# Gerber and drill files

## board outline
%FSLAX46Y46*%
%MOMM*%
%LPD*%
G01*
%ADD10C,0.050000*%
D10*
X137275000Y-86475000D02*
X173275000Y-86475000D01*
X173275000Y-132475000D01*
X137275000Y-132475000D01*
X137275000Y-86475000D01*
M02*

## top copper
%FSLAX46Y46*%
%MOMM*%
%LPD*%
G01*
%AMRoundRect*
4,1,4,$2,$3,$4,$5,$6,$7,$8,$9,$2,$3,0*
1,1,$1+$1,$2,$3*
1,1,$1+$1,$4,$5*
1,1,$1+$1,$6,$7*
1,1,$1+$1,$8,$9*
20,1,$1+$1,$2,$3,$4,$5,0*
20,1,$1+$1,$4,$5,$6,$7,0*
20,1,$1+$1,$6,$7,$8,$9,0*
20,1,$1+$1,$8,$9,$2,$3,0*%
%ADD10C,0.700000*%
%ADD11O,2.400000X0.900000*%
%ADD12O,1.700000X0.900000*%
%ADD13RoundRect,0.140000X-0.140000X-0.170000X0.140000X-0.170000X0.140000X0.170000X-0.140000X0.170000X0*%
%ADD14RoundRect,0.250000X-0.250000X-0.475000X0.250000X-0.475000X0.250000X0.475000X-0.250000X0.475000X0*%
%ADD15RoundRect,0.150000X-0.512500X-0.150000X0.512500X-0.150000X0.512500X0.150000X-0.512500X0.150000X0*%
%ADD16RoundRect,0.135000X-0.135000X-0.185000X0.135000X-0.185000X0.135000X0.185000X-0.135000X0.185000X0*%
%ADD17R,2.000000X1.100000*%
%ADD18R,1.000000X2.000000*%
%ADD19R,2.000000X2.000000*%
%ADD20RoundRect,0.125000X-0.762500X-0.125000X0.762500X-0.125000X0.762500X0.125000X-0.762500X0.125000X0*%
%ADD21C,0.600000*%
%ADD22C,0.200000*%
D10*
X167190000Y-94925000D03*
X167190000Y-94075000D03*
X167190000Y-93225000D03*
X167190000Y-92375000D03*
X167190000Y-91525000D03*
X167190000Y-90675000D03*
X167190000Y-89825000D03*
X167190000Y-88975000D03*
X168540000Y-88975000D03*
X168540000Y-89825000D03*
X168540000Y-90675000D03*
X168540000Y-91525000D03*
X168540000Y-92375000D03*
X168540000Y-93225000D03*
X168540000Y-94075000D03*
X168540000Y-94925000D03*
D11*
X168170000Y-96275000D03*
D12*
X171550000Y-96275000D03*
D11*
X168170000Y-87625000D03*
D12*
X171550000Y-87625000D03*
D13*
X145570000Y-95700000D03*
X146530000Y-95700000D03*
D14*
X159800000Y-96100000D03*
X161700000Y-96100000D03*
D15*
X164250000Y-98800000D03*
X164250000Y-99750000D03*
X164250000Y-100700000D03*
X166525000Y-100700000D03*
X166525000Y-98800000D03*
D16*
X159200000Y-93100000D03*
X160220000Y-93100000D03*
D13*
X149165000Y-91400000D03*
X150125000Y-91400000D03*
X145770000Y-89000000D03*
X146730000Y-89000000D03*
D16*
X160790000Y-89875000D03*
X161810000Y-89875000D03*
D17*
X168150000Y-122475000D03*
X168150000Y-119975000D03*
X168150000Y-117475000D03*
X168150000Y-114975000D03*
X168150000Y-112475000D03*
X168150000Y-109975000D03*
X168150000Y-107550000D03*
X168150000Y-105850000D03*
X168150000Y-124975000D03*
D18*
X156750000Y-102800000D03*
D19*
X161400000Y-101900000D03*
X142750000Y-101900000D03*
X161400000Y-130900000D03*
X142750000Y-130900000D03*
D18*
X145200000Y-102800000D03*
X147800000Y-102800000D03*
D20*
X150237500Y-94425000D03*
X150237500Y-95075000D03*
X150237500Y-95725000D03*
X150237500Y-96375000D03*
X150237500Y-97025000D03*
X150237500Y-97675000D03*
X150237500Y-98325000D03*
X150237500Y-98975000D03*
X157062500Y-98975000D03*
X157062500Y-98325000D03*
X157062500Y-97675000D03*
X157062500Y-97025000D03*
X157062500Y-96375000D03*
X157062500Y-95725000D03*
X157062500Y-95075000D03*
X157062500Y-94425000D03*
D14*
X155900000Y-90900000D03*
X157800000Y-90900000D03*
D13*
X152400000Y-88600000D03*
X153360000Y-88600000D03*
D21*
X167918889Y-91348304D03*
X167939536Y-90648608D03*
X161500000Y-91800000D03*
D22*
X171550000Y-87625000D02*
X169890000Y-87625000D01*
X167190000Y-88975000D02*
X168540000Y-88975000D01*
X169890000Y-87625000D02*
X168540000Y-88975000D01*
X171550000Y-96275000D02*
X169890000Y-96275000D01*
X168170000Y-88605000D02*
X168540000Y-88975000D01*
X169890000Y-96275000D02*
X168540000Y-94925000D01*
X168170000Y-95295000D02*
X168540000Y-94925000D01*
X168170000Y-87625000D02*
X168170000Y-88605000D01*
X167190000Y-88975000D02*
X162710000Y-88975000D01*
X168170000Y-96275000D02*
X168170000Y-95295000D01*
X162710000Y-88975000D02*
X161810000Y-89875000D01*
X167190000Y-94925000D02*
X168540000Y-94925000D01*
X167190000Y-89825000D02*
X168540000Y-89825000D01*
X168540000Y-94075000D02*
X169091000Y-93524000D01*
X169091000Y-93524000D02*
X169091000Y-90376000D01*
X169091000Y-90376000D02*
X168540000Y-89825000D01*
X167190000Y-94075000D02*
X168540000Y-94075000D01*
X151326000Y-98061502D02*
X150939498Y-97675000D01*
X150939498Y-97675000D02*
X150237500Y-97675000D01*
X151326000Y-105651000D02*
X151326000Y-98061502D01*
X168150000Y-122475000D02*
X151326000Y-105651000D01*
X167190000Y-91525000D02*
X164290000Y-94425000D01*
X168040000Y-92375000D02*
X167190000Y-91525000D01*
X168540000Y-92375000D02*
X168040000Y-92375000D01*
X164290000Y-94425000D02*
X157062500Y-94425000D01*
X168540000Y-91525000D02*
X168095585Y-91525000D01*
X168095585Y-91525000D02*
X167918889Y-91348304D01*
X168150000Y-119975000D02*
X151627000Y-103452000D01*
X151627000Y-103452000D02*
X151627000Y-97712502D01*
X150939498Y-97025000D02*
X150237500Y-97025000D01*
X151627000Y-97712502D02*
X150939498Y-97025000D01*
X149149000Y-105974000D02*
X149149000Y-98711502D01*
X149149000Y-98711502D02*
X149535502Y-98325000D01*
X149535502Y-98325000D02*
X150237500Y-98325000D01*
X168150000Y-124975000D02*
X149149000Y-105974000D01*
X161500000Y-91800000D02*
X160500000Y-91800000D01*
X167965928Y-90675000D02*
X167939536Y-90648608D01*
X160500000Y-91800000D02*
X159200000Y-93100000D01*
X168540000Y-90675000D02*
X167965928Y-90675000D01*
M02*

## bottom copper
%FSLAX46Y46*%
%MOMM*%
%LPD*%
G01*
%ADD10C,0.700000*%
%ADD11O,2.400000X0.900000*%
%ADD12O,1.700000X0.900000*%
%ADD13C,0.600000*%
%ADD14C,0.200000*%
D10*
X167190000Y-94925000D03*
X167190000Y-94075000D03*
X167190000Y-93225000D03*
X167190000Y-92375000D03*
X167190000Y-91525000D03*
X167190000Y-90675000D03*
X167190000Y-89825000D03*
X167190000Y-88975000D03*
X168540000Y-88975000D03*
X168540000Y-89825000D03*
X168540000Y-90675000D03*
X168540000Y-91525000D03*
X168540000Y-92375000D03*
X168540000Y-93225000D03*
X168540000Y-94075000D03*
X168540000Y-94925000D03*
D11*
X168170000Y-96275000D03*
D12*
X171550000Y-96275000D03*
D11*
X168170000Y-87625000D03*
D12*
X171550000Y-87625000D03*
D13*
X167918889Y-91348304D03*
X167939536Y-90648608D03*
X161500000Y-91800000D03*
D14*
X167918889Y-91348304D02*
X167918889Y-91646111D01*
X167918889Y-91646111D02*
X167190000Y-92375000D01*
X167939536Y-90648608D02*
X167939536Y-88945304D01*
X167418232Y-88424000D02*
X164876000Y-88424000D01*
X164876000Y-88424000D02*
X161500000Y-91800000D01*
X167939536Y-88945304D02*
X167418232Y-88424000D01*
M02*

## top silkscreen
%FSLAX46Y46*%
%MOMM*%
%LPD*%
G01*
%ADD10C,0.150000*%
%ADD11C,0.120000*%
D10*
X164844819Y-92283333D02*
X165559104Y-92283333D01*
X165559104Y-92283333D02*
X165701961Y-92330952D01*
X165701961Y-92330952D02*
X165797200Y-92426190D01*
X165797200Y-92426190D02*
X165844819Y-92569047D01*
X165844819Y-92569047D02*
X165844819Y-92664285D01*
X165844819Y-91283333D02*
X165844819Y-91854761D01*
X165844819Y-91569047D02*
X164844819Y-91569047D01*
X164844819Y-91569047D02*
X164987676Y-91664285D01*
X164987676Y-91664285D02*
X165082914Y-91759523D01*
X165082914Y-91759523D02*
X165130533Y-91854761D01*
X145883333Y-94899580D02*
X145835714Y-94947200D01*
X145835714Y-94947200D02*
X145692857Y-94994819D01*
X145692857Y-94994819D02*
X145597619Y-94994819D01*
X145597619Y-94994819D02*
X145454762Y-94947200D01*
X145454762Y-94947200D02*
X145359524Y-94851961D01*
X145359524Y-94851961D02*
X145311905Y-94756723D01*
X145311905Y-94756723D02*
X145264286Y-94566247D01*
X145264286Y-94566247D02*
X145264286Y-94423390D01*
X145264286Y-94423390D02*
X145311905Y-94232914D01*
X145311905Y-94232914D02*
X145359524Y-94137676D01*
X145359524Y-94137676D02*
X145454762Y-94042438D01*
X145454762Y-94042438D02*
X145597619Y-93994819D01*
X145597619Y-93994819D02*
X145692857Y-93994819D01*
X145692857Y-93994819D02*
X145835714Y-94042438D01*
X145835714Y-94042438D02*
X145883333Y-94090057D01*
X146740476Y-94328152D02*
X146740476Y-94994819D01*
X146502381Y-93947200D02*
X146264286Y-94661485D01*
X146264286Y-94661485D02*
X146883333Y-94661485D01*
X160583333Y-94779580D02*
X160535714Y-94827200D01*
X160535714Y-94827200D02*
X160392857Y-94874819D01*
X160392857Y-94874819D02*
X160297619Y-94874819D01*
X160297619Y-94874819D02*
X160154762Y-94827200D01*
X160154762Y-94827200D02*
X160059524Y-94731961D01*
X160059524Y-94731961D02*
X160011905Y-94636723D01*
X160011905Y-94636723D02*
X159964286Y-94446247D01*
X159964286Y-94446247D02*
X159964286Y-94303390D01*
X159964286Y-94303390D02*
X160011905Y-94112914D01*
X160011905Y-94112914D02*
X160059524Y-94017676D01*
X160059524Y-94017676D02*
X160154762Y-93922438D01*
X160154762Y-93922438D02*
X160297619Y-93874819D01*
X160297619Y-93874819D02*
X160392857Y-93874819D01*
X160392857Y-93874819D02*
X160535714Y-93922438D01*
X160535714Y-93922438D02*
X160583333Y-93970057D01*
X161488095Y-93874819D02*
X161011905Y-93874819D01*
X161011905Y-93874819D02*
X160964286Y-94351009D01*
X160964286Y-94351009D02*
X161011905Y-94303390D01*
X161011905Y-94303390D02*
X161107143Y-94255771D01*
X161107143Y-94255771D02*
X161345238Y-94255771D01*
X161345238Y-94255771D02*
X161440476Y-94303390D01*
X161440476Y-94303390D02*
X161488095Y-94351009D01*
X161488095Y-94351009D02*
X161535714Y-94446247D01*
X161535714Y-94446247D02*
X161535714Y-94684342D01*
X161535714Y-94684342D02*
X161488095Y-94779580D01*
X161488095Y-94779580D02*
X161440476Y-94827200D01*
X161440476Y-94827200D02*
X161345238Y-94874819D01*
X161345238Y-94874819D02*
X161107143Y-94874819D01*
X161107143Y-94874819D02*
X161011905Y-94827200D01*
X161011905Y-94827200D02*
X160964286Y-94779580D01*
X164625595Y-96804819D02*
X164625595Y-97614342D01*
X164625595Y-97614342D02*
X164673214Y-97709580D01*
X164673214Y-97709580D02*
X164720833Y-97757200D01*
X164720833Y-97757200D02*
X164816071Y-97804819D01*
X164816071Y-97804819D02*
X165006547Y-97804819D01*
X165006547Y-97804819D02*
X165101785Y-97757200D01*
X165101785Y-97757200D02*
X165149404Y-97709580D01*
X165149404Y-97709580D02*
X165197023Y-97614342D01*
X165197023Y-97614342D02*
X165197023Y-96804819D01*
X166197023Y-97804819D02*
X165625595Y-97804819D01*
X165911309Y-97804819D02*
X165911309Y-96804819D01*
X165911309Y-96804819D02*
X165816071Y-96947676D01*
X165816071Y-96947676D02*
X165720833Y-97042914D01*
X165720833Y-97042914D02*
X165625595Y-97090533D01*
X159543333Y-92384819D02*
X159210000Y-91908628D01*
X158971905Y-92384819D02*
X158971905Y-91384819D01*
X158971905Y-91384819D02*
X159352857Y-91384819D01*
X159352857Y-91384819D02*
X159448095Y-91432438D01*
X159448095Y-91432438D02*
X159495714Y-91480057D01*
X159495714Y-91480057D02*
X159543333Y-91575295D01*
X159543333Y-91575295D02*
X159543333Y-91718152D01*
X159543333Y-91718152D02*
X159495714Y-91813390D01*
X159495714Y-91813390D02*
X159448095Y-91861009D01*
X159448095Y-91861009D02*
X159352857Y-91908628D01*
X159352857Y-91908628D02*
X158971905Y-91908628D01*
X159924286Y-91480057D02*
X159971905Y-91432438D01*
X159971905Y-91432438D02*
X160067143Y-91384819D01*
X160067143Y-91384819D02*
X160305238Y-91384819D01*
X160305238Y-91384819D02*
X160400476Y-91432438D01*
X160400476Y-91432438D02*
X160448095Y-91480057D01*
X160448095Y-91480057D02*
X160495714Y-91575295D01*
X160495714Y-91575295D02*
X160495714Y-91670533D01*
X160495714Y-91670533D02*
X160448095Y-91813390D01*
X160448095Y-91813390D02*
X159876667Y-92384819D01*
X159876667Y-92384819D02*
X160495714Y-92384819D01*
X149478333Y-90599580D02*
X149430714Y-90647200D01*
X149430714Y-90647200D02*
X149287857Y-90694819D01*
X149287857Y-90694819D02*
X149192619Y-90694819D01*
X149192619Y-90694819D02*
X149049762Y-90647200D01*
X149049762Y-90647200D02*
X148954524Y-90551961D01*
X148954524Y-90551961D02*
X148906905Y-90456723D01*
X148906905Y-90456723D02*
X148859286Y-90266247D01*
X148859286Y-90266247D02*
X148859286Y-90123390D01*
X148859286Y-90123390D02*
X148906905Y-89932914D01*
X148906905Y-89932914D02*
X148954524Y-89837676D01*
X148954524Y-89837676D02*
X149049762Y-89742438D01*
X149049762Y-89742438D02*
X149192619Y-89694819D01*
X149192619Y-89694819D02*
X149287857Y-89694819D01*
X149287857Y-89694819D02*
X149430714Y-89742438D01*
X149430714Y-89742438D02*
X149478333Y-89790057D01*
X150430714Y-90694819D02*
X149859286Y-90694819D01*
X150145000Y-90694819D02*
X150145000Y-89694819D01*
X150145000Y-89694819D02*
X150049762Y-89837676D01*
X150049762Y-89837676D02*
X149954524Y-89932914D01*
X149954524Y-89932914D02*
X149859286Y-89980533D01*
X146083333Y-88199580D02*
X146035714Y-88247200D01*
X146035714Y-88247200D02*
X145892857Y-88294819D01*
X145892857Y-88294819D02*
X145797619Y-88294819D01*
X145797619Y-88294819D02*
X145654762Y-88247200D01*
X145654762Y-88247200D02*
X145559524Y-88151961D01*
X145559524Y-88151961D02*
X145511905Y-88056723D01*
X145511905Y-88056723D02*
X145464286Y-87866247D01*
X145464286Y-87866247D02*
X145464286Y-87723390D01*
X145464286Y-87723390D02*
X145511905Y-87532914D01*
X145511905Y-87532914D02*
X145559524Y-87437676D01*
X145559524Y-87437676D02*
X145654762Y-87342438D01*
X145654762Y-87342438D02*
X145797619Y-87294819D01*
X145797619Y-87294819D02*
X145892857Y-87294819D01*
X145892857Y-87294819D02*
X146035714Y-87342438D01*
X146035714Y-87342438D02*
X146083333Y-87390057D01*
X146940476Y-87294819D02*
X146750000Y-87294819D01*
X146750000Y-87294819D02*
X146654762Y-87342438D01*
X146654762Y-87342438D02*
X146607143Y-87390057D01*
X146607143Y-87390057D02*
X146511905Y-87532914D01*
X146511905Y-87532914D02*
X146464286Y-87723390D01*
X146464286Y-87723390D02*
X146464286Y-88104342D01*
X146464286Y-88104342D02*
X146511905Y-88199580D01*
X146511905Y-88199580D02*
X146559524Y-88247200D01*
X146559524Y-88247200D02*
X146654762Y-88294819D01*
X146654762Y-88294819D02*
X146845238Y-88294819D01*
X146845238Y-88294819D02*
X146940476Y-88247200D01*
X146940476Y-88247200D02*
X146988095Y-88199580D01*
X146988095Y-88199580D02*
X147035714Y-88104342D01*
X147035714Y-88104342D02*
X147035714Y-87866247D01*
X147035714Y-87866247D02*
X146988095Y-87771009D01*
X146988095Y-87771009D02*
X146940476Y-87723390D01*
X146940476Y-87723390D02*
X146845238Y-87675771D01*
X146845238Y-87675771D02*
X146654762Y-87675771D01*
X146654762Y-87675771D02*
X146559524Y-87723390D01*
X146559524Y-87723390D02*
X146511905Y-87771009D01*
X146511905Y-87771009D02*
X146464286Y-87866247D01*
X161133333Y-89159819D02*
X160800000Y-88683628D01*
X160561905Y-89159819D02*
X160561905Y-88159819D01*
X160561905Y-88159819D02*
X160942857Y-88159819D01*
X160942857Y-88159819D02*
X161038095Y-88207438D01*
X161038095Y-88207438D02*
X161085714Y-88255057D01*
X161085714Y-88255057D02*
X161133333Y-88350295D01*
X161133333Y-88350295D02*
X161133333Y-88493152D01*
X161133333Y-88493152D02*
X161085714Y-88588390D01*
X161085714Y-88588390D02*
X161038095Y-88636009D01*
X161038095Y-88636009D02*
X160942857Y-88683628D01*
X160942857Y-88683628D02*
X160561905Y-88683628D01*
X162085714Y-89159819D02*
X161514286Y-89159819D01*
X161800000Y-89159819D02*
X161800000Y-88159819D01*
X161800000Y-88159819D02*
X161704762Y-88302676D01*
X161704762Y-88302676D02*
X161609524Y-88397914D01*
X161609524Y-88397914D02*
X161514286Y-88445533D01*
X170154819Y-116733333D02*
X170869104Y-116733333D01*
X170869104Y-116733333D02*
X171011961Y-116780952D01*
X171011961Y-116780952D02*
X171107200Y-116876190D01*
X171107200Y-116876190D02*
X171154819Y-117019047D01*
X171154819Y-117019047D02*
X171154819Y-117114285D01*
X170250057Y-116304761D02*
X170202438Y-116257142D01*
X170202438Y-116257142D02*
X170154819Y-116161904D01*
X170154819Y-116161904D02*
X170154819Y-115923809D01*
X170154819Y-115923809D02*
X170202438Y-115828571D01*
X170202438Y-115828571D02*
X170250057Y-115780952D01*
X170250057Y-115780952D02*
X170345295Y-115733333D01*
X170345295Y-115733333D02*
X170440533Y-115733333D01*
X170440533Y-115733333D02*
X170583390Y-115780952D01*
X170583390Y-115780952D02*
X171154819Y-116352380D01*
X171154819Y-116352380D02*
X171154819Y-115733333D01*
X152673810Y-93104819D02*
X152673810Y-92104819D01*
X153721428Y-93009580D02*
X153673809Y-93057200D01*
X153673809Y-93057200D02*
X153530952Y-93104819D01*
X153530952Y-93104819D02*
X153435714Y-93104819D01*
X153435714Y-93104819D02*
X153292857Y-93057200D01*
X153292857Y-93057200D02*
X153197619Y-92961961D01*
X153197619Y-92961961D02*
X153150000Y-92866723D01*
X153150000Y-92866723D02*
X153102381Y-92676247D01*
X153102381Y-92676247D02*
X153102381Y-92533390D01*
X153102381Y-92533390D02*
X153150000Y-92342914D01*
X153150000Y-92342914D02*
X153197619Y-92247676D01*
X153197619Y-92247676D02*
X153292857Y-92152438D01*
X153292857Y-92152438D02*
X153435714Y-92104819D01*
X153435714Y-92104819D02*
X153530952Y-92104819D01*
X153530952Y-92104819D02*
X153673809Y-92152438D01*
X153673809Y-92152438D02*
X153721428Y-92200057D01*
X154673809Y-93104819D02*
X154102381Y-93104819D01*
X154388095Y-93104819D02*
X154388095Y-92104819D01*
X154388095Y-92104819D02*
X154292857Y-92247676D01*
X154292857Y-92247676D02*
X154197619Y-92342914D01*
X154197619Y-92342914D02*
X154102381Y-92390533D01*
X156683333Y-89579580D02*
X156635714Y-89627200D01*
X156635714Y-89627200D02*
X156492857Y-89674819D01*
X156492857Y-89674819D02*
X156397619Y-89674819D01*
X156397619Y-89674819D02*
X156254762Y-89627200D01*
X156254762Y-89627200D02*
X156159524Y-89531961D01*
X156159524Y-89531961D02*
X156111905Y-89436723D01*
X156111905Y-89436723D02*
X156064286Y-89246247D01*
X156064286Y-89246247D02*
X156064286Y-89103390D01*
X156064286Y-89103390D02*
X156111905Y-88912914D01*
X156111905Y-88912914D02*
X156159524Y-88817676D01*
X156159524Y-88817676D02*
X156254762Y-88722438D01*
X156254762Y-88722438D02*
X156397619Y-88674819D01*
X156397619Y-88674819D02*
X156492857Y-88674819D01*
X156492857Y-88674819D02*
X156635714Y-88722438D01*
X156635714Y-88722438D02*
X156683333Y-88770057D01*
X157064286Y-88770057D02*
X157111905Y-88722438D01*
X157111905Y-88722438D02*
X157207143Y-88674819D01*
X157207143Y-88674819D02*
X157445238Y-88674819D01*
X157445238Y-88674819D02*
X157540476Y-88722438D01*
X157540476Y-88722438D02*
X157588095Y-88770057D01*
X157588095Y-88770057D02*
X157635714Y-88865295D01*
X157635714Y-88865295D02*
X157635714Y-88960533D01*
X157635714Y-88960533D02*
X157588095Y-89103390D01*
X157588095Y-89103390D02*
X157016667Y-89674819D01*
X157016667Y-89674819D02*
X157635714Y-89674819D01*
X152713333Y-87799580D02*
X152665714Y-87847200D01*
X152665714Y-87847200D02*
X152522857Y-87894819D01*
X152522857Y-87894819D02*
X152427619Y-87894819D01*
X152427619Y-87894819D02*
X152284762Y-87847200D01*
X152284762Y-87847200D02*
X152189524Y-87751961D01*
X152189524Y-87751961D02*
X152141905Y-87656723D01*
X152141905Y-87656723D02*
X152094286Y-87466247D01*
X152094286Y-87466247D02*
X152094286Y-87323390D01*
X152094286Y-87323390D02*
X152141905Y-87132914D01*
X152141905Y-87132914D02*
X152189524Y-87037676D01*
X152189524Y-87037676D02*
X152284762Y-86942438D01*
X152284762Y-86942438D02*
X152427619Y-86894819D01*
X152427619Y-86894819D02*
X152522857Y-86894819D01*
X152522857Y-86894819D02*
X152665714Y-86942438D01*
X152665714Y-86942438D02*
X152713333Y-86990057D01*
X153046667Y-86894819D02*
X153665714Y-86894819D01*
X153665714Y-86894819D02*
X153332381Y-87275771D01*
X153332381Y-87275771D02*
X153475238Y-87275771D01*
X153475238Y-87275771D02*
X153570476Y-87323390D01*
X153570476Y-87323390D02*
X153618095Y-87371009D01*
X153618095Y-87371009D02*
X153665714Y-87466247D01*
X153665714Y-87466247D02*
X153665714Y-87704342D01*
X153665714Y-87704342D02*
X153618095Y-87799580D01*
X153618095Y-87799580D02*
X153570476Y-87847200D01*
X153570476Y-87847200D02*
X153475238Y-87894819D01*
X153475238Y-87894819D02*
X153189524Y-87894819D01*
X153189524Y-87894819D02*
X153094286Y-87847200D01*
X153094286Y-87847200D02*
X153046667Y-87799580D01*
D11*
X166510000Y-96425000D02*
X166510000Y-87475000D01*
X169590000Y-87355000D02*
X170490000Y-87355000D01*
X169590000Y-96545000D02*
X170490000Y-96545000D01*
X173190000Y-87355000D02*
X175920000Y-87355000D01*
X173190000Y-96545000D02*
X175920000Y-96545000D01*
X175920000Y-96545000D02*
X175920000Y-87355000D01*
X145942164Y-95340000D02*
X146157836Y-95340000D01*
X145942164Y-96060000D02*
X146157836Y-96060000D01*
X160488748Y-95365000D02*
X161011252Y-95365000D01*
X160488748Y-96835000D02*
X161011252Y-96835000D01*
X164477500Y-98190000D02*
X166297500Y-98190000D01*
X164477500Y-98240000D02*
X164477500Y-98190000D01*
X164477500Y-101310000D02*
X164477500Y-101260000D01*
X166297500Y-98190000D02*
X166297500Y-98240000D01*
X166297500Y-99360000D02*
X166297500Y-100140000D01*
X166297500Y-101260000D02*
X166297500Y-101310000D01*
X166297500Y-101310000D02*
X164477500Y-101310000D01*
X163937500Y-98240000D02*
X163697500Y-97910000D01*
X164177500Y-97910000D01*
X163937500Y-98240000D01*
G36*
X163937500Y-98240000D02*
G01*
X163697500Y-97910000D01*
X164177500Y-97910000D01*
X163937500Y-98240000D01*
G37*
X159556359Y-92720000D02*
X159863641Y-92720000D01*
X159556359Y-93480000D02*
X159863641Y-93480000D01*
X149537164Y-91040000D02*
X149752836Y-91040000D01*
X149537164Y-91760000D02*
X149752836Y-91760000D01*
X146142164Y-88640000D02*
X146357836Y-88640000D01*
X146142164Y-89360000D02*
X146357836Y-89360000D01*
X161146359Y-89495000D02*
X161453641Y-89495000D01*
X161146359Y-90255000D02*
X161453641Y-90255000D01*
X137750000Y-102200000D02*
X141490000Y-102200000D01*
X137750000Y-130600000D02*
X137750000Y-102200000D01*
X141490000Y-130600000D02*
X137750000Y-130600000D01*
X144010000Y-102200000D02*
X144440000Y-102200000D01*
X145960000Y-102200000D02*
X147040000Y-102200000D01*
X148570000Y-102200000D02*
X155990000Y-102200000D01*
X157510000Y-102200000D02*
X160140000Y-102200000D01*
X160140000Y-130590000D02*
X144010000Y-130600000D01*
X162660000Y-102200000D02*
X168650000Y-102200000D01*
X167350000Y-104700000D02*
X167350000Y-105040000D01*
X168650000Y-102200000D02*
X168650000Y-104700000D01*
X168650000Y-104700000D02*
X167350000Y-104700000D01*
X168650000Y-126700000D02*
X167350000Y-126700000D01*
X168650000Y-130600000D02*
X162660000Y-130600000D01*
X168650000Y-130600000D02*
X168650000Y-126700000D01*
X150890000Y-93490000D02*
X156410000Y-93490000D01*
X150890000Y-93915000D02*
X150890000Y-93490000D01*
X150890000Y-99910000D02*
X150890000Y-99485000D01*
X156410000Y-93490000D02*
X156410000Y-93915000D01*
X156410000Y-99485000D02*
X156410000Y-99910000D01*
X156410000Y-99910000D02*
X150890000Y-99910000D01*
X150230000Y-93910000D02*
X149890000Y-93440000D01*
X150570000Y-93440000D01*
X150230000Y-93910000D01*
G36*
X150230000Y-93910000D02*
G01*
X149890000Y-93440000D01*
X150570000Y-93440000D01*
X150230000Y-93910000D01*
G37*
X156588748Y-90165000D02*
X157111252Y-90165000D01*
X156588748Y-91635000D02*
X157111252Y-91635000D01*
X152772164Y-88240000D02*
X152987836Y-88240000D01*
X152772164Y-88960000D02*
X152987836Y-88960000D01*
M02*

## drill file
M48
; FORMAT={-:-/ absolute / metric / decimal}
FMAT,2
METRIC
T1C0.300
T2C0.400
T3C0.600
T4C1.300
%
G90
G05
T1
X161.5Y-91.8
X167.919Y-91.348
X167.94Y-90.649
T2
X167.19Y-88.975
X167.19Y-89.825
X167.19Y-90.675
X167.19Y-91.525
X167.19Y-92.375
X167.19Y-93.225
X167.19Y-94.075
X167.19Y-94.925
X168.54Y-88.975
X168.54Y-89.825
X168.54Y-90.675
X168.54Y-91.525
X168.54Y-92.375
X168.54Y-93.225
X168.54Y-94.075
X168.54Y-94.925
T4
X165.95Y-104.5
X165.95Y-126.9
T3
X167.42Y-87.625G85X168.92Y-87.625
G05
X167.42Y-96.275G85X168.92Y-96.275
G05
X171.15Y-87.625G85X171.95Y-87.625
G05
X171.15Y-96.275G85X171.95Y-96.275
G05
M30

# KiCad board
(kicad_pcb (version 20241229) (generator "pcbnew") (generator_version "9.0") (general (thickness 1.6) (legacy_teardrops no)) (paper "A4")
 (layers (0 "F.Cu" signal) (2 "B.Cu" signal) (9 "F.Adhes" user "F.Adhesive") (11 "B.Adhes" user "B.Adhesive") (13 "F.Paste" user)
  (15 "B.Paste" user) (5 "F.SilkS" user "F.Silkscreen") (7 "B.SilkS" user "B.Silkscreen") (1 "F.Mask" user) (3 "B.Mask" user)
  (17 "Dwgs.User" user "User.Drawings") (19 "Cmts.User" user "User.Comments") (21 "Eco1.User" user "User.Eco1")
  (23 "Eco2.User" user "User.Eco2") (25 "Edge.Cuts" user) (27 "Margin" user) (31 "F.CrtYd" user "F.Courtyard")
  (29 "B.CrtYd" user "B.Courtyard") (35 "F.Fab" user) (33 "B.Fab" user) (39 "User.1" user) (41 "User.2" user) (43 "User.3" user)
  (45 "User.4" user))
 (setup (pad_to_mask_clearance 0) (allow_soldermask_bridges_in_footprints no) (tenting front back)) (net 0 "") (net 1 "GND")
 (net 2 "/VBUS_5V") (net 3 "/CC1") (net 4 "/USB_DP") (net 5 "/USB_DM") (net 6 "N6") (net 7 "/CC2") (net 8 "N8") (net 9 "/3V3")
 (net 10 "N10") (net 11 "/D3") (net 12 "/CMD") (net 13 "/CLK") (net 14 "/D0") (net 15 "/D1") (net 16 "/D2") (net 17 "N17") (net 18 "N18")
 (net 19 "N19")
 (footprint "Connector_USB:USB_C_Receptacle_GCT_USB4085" (layer "F.Cu") (at 167.19 94.925 90)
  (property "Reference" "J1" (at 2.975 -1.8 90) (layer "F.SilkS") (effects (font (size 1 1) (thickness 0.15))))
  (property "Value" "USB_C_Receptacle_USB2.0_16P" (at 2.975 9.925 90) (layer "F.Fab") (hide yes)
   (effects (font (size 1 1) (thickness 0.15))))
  (fp_line (start -1.5 -0.68) (end 7.45 -0.68) (stroke (width 0.12) (type solid)) (layer "F.SilkS"))
  (fp_line (start 7.57 2.4) (end 7.57 3.3) (stroke (width 0.12) (type solid)) (layer "F.SilkS"))
  (fp_line (start -1.62 2.4) (end -1.62 3.3) (stroke (width 0.12) (type solid)) (layer "F.SilkS"))
  (fp_line (start 7.57 6) (end 7.57 8.73) (stroke (width 0.12) (type solid)) (layer "F.SilkS"))
  (fp_line (start -1.62 6) (end -1.62 8.73) (stroke (width 0.12) (type solid)) (layer "F.SilkS"))
  (fp_line (start -1.62 8.73) (end 7.57 8.73) (stroke (width 0.12) (type solid)) (layer "F.SilkS"))
  (pad "A1" thru_hole circle (at 0 0 90) (size 0.7 0.7) (drill 0.4) (layers "*.Cu" "*.Mask") (remove_unused_layers no) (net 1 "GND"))
  (pad "A4" thru_hole circle (at 0.85 0 90) (size 0.7 0.7) (drill 0.4) (layers "*.Cu" "*.Mask") (remove_unused_layers no) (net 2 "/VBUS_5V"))
  (pad "A5" thru_hole circle (at 1.7 0 90) (size 0.7 0.7) (drill 0.4) (layers "*.Cu" "*.Mask") (remove_unused_layers no) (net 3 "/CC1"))
  (pad "A6" thru_hole circle (at 2.55 0 90) (size 0.7 0.7) (drill 0.4) (layers "*.Cu" "*.Mask") (remove_unused_layers no) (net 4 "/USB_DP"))
  (pad "A7" thru_hole circle (at 3.4 0 90) (size 0.7 0.7) (drill 0.4) (layers "*.Cu" "*.Mask") (remove_unused_layers no) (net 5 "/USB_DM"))
  (pad "A8" thru_hole circle (at 4.25 0 90) (size 0.7 0.7) (drill 0.4) (layers "*.Cu" "*.Mask") (remove_unused_layers no) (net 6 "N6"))
  (pad "A9" thru_hole circle (at 5.1 0 90) (size 0.7 0.7) (drill 0.4) (layers "*.Cu" "*.Mask") (remove_unused_layers no) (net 2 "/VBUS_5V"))
  (pad "A12" thru_hole circle (at 5.95 0 90) (size 0.7 0.7) (drill 0.4) (layers "*.Cu" "*.Mask") (remove_unused_layers no) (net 1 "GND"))
  (pad "B1" thru_hole circle (at 5.95 1.35 90) (size 0.7 0.7) (drill 0.4) (layers "*.Cu" "*.Mask") (remove_unused_layers no) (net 1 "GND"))
  (pad "B4" thru_hole circle (at 5.1 1.35 90) (size 0.7 0.7) (drill 0.4) (layers "*.Cu" "*.Mask") (remove_unused_layers no)
   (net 2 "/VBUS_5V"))
  (pad "B5" thru_hole circle (at 4.25 1.35 90) (size 0.7 0.7) (drill 0.4) (layers "*.Cu" "*.Mask") (remove_unused_layers no) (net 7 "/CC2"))
  (pad "B6" thru_hole circle (at 3.4 1.35 90) (size 0.7 0.7) (drill 0.4) (layers "*.Cu" "*.Mask") (remove_unused_layers no)
   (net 4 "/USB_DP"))
  (pad "B7" thru_hole circle (at 2.55 1.35 90) (size 0.7 0.7) (drill 0.4) (layers "*.Cu" "*.Mask") (remove_unused_layers no)
   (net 5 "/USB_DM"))
  (pad "B8" thru_hole circle (at 1.7 1.35 90) (size 0.7 0.7) (drill 0.4) (layers "*.Cu" "*.Mask") (remove_unused_layers no) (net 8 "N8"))
  (pad "B9" thru_hole circle (at 0.85 1.35 90) (size 0.7 0.7) (drill 0.4) (layers "*.Cu" "*.Mask") (remove_unused_layers no)
   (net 2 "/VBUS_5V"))
  (pad "B12" thru_hole circle (at 0 1.35 90) (size 0.7 0.7) (drill 0.4) (layers "*.Cu" "*.Mask") (remove_unused_layers no) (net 1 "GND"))
  (pad "S1" thru_hole oval (at -1.35 0.98 90) (size 0.9 2.4) (drill oval 0.6 2.1) (layers "*.Cu" "*.Mask") (remove_unused_layers no)
   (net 1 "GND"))
  (pad "S1" thru_hole oval (at -1.35 4.36 90) (size 0.9 1.7) (drill oval 0.6 1.4) (layers "*.Cu" "*.Mask") (remove_unused_layers no)
   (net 1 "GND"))
  (pad "S1" thru_hole oval (at 7.3 0.98 90) (size 0.9 2.4) (drill oval 0.6 2.1) (layers "*.Cu" "*.Mask") (remove_unused_layers no)
   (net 1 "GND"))
  (pad "S1" thru_hole oval (at 7.3 4.36 90) (size 0.9 1.7) (drill oval 0.6 1.4) (layers "*.Cu" "*.Mask") (remove_unused_layers no)
   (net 1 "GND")))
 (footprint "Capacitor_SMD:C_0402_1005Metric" (layer "F.Cu") (at 146.05 95.7)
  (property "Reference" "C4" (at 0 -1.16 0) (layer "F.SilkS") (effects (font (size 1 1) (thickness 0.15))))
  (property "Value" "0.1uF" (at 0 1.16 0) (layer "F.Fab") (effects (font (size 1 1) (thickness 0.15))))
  (fp_line (start -0.107836 -0.36) (end 0.107836 -0.36) (stroke (width 0.12) (type solid)) (layer "F.SilkS"))
  (fp_line (start -0.107836 0.36) (end 0.107836 0.36) (stroke (width 0.12) (type solid)) (layer "F.SilkS"))
  (pad "1" smd roundrect (at -0.48 0) (size 0.56 0.62) (layers "F.Cu" "F.Mask" "F.Paste") (roundrect_rratio 0.25) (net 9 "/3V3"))
  (pad "2" smd roundrect (at 0.48 0) (size 0.56 0.62) (layers "F.Cu" "F.Mask" "F.Paste") (roundrect_rratio 0.25) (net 1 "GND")))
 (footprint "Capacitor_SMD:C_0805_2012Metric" (layer "F.Cu") (at 160.75 96.1)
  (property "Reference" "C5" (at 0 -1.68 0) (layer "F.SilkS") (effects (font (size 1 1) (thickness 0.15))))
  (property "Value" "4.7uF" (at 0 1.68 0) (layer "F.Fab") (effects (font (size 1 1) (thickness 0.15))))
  (fp_line (start -0.261252 -0.735) (end 0.261252 -0.735) (stroke (width 0.12) (type solid)) (layer "F.SilkS"))
  (fp_line (start -0.261252 0.735) (end 0.261252 0.735) (stroke (width 0.12) (type solid)) (layer "F.SilkS"))
  (pad "1" smd roundrect (at -0.95 0) (size 1 1.45) (layers "F.Cu" "F.Mask" "F.Paste") (roundrect_rratio 0.25) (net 9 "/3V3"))
  (pad "2" smd roundrect (at 0.95 0) (size 1 1.45) (layers "F.Cu" "F.Mask" "F.Paste") (roundrect_rratio 0.25) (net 1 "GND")))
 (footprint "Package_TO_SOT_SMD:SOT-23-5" (layer "F.Cu") (at 165.3875 99.75)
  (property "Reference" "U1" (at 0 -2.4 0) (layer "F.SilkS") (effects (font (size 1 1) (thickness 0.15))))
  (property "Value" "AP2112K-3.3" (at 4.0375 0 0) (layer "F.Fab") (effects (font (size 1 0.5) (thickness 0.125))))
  (fp_line (start -0.91 -1.56) (end 0.91 -1.56) (stroke (width 0.12) (type solid)) (layer "F.SilkS"))
  (fp_line (start -0.91 -1.51) (end -0.91 -1.56) (stroke (width 0.12) (type solid)) (layer "F.SilkS"))
  (fp_line (start -0.91 1.56) (end -0.91 1.51) (stroke (width 0.12) (type solid)) (layer "F.SilkS"))
  (fp_line (start 0.91 -1.56) (end 0.91 -1.51) (stroke (width 0.12) (type solid)) (layer "F.SilkS"))
  (fp_line (start 0.91 -0.39) (end 0.91 0.39) (stroke (width 0.12) (type solid)) (layer "F.SilkS"))
  (fp_line (start 0.91 1.51) (end 0.91 1.56) (stroke (width 0.12) (type solid)) (layer "F.SilkS"))
  (fp_line (start 0.91 1.56) (end -0.91 1.56) (stroke (width 0.12) (type solid)) (layer "F.SilkS"))
  (fp_poly (pts (xy -1.45 -1.51) (xy -1.69 -1.84) (xy -1.21 -1.84)) (stroke (width 0.12) (type solid)) (fill yes) (layer "F.SilkS"))
  (pad "1" smd roundrect (at -1.1375 -0.95) (size 1.325 0.6) (layers "F.Cu" "F.Mask" "F.Paste") (roundrect_rratio 0.25) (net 2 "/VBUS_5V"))
  (pad "2" smd roundrect (at -1.1375 0) (size 1.325 0.6) (layers "F.Cu" "F.Mask" "F.Paste") (roundrect_rratio 0.25) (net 1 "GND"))
  (pad "3" smd roundrect (at -1.1375 0.95) (size 1.325 0.6) (layers "F.Cu" "F.Mask" "F.Paste") (roundrect_rratio 0.25) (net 2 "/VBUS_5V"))
  (pad "4" smd roundrect (at 1.1375 0.95) (size 1.325 0.6) (layers "F.Cu" "F.Mask" "F.Paste") (roundrect_rratio 0.25) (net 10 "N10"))
  (pad "5" smd roundrect (at 1.1375 -0.95) (size 1.325 0.6) (layers "F.Cu" "F.Mask" "F.Paste") (roundrect_rratio 0.25) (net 9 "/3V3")))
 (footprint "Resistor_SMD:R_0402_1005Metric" (layer "F.Cu") (at 159.71 93.1)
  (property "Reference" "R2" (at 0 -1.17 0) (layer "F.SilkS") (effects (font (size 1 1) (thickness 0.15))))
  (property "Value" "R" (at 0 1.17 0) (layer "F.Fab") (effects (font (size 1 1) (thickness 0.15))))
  (fp_line (start -0.153641 -0.38) (end 0.153641 -0.38) (stroke (width 0.12) (type solid)) (layer "F.SilkS"))
  (fp_line (start -0.153641 0.38) (end 0.153641 0.38) (stroke (width 0.12) (type solid)) (layer "F.SilkS"))
  (pad "1" smd roundrect (at -0.51 0) (size 0.54 0.64) (layers "F.Cu" "F.Mask" "F.Paste") (roundrect_rratio 0.25) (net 7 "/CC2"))
  (pad "2" smd roundrect (at 0.51 0) (size 0.54 0.64) (layers "F.Cu" "F.Mask" "F.Paste") (roundrect_rratio 0.25) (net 1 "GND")))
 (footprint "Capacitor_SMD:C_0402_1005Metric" (layer "F.Cu") (at 149.645 91.4)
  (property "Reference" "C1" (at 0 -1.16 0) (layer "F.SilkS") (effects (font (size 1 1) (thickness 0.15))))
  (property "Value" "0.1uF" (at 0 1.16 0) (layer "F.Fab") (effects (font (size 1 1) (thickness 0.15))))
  (fp_line (start -0.107836 -0.36) (end 0.107836 -0.36) (stroke (width 0.12) (type solid)) (layer "F.SilkS"))
  (fp_line (start -0.107836 0.36) (end 0.107836 0.36) (stroke (width 0.12) (type solid)) (layer "F.SilkS"))
  (pad "1" smd roundrect (at -0.48 0) (size 0.56 0.62) (layers "F.Cu" "F.Mask" "F.Paste") (roundrect_rratio 0.25) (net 2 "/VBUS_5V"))
  (pad "2" smd roundrect (at 0.48 0) (size 0.56 0.62) (layers "F.Cu" "F.Mask" "F.Paste") (roundrect_rratio 0.25) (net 1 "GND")))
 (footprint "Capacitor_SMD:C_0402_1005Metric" (layer "F.Cu") (at 146.25 89)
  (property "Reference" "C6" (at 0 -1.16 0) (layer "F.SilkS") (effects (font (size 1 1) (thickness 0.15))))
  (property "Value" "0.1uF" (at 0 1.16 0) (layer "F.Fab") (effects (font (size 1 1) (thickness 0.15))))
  (fp_line (start -0.107836 -0.36) (end 0.107836 -0.36) (stroke (width 0.12) (type solid)) (layer "F.SilkS"))
  (fp_line (start -0.107836 0.36) (end 0.107836 0.36) (stroke (width 0.12) (type solid)) (layer "F.SilkS"))
  (pad "1" smd roundrect (at -0.48 0) (size 0.56 0.62) (layers "F.Cu" "F.Mask" "F.Paste") (roundrect_rratio 0.25) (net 9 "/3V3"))
  (pad "2" smd roundrect (at 0.48 0) (size 0.56 0.62) (layers "F.Cu" "F.Mask" "F.Paste") (roundrect_rratio 0.25) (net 1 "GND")))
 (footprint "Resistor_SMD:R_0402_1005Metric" (layer "F.Cu") (at 161.3 89.875)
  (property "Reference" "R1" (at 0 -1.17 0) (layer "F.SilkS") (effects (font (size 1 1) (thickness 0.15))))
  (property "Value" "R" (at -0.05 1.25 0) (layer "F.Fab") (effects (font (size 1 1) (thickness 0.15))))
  (fp_line (start -0.153641 -0.38) (end 0.153641 -0.38) (stroke (width 0.12) (type solid)) (layer "F.SilkS"))
  (fp_line (start -0.153641 0.38) (end 0.153641 0.38) (stroke (width 0.12) (type solid)) (layer "F.SilkS"))
  (pad "1" smd roundrect (at -0.51 0) (size 0.54 0.64) (layers "F.Cu" "F.Mask" "F.Paste") (roundrect_rratio 0.25) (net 3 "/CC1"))
  (pad "2" smd roundrect (at 0.51 0) (size 0.54 0.64) (layers "F.Cu" "F.Mask" "F.Paste") (roundrect_rratio 0.25) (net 1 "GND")))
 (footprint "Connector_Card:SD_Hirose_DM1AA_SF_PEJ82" (layer "F.Cu") (at 153.2 116.4 -90)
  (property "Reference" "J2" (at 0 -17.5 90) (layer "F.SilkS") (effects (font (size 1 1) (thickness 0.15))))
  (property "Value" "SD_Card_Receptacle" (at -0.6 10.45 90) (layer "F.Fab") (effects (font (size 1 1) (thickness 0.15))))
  (fp_line (start -14.2 15.45) (end -14.2 11.71) (stroke (width 0.12) (type solid)) (layer "F.SilkS"))
  (fp_line (start 14.2 15.45) (end -14.2 15.45) (stroke (width 0.12) (type solid)) (layer "F.SilkS"))
  (fp_line (start 14.2 11.71) (end 14.2 15.45) (stroke (width 0.12) (type solid)) (layer "F.SilkS"))
  (fp_line (start -14.2 9.19) (end -14.2 8.76) (stroke (width 0.12) (type solid)) (layer "F.SilkS"))
  (fp_line (start -14.2 7.24) (end -14.2 6.16) (stroke (width 0.12) (type solid)) (layer "F.SilkS"))
  (fp_line (start -14.2 4.63) (end -14.2 -2.79) (stroke (width 0.12) (type solid)) (layer "F.SilkS"))
  (fp_line (start -14.2 -4.31) (end -14.2 -6.94) (stroke (width 0.12) (type solid)) (layer "F.SilkS"))
  (fp_line (start 14.19 -6.94) (end 14.2 9.19) (stroke (width 0.12) (type solid)) (layer "F.SilkS"))
  (fp_line (start -14.2 -9.46) (end -14.2 -15.45) (stroke (width 0.12) (type solid)) (layer "F.SilkS"))
  (fp_line (start -11.7 -14.15) (end -11.36 -14.15) (stroke (width 0.12) (type solid)) (layer "F.SilkS"))
  (fp_line (start -14.2 -15.45) (end -11.7 -15.45) (stroke (width 0.12) (type solid)) (layer "F.SilkS"))
  (fp_line (start -11.7 -15.45) (end -11.7 -14.15) (stroke (width 0.12) (type solid)) (layer "F.SilkS"))
  (fp_line (start 10.3 -15.45) (end 10.3 -14.15) (stroke (width 0.12) (type solid)) (layer "F.SilkS"))
  (fp_line (start 14.2 -15.45) (end 14.2 -9.46) (stroke (width 0.12) (type solid)) (layer "F.SilkS"))
  (fp_line (start 14.2 -15.45) (end 10.3 -15.45) (stroke (width 0.12) (type solid)) (layer "F.SilkS"))
  (pad "" np_thru_hole circle (at -11.9 -12.75 270) (size 1.3 1.3) (drill 1.3) (layers "*.Cu" "*.Mask"))
  (pad "" np_thru_hole circle (at 10.5 -12.75 270) (size 1.3 1.3) (drill 1.3) (layers "*.Cu" "*.Mask"))
  (pad "1" smd rect (at 6.075 -14.95 270) (size 1.1 2) (layers "F.Cu" "F.Mask" "F.Paste") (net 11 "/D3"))
  (pad "2" smd rect (at 3.575 -14.95 270) (size 1.1 2) (layers "F.Cu" "F.Mask" "F.Paste") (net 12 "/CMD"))
  (pad "3" smd rect (at 1.075 -14.95 270) (size 1.1 2) (layers "F.Cu" "F.Mask" "F.Paste") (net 1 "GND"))
  (pad "4" smd rect (at -1.425 -14.95 270) (size 1.1 2) (layers "F.Cu" "F.Mask" "F.Paste") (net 9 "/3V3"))
  (pad "5" smd rect (at -3.925 -14.95 270) (size 1.1 2) (layers "F.Cu" "F.Mask" "F.Paste") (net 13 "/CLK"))
  (pad "6" smd rect (at -6.425 -14.95 270) (size 1.1 2) (layers "F.Cu" "F.Mask" "F.Paste") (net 1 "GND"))
  (pad "7" smd rect (at -8.85 -14.95 270) (size 1.1 2) (layers "F.Cu" "F.Mask" "F.Paste") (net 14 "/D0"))
  (pad "8" smd rect (at -10.55 -14.95 270) (size 1.1 2) (layers "F.Cu" "F.Mask" "F.Paste") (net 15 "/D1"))
  (pad "9" smd rect (at 8.575 -14.95 270) (size 1.1 2) (layers "F.Cu" "F.Mask" "F.Paste") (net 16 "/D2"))
  (pad "CP" smd rect (at -13.6 -3.55 270) (size 2 1) (layers "F.Cu" "F.Mask" "F.Paste"))
  (pad "SH" smd rect (at -14.5 -8.2 270) (size 2 2) (layers "F.Cu" "F.Mask" "F.Paste"))
  (pad "SH" smd rect (at -14.5 10.45 270) (size 2 2) (layers "F.Cu" "F.Mask" "F.Paste"))
  (pad "SH" smd rect (at 14.5 -8.2 270) (size 2 2) (layers "F.Cu" "F.Mask" "F.Paste"))
  (pad "SH" smd rect (at 14.5 10.45 270) (size 2 2) (layers "F.Cu" "F.Mask" "F.Paste"))
  (pad "SW" smd rect (at -13.6 8 270) (size 2 1) (layers "F.Cu" "F.Mask" "F.Paste"))
  (pad "WP" smd rect (at -13.6 5.4 270) (size 2 1) (layers "F.Cu" "F.Mask" "F.Paste")))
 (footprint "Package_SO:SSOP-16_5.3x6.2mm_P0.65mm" (layer "F.Cu") (at 153.65 96.7)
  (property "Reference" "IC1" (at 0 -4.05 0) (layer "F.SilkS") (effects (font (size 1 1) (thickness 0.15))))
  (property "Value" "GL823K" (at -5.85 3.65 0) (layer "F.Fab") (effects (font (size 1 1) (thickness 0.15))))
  (fp_line (start -2.76 -3.21) (end 2.76 -3.21) (stroke (width 0.12) (type solid)) (layer "F.SilkS"))
  (fp_line (start -2.76 -2.785) (end -2.76 -3.21) (stroke (width 0.12) (type solid)) (layer "F.SilkS"))
  (fp_line (start -2.76 3.21) (end -2.76 2.785) (stroke (width 0.12) (type solid)) (layer "F.SilkS"))
  (fp_line (start 2.76 -3.21) (end 2.76 -2.785) (stroke (width 0.12) (type solid)) (layer "F.SilkS"))
  (fp_line (start 2.76 2.785) (end 2.76 3.21) (stroke (width 0.12) (type solid)) (layer "F.SilkS"))
  (fp_line (start 2.76 3.21) (end -2.76 3.21) (stroke (width 0.12) (type solid)) (layer "F.SilkS"))
  (fp_poly (pts (xy -3.42 -2.79) (xy -3.76 -3.26) (xy -3.08 -3.26)) (stroke (width 0.12) (type solid)) (fill yes) (layer "F.SilkS"))
  (pad "1" smd roundrect (at -3.4125 -2.275) (size 1.775 0.5) (layers "F.Cu" "F.Mask" "F.Paste") (roundrect_rratio 0.25) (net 1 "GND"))
  (pad "2" smd roundrect (at -3.4125 -1.625) (size 1.775 0.5) (layers "F.Cu" "F.Mask" "F.Paste") (roundrect_rratio 0.25) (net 15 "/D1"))
  (pad "3" smd roundrect (at -3.4125 -0.975) (size 1.775 0.5) (layers "F.Cu" "F.Mask" "F.Paste") (roundrect_rratio 0.25) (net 14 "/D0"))
  (pad "4" smd roundrect (at -3.4125 -0.325) (size 1.775 0.5) (layers "F.Cu" "F.Mask" "F.Paste") (roundrect_rratio 0.25) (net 13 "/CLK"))
  (pad "5" smd roundrect (at -3.4125 0.325) (size 1.775 0.5) (layers "F.Cu" "F.Mask" "F.Paste") (roundrect_rratio 0.25) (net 12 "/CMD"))
  (pad "6" smd roundrect (at -3.4125 0.975) (size 1.775 0.5) (layers "F.Cu" "F.Mask" "F.Paste") (roundrect_rratio 0.25) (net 11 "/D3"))
  (pad "7" smd roundrect (at -3.4125 1.625) (size 1.775 0.5) (layers "F.Cu" "F.Mask" "F.Paste") (roundrect_rratio 0.25) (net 16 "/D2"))
  (pad "8" smd roundrect (at -3.4125 2.275) (size 1.775 0.5) (layers "F.Cu" "F.Mask" "F.Paste") (roundrect_rratio 0.25) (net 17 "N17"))
  (pad "9" smd roundrect (at 3.4125 2.275) (size 1.775 0.5) (layers "F.Cu" "F.Mask" "F.Paste") (roundrect_rratio 0.25) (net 9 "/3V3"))
  (pad "10" smd roundrect (at 3.4125 1.625) (size 1.775 0.5) (layers "F.Cu" "F.Mask" "F.Paste") (roundrect_rratio 0.25) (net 2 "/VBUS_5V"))
  (pad "11" smd roundrect (at 3.4125 0.975) (size 1.775 0.5) (layers "F.Cu" "F.Mask" "F.Paste") (roundrect_rratio 0.25) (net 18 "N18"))
  (pad "12" smd roundrect (at 3.4125 0.325) (size 1.775 0.5) (layers "F.Cu" "F.Mask" "F.Paste") (roundrect_rratio 0.25) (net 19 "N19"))
  (pad "13" smd roundrect (at 3.4125 -0.325) (size 1.775 0.5) (layers "F.Cu" "F.Mask" "F.Paste") (roundrect_rratio 0.25) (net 9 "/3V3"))
  (pad "14" smd roundrect (at 3.4125 -0.975) (size 1.775 0.5) (layers "F.Cu" "F.Mask" "F.Paste") (roundrect_rratio 0.25) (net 1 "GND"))
  (pad "15" smd roundrect (at 3.4125 -1.625) (size 1.775 0.5) (layers "F.Cu" "F.Mask" "F.Paste") (roundrect_rratio 0.25) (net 4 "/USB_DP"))
  (pad "16" smd roundrect (at 3.4125 -2.275) (size 1.775 0.5) (layers "F.Cu" "F.Mask" "F.Paste") (roundrect_rratio 0.25) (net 5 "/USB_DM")))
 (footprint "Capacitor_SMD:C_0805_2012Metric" (layer "F.Cu") (at 156.85 90.9)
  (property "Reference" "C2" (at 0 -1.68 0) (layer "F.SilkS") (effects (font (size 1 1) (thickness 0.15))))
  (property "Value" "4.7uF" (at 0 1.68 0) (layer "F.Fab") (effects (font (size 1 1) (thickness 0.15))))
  (fp_line (start -0.261252 -0.735) (end 0.261252 -0.735) (stroke (width 0.12) (type solid)) (layer "F.SilkS"))
  (fp_line (start -0.261252 0.735) (end 0.261252 0.735) (stroke (width 0.12) (type solid)) (layer "F.SilkS"))
  (pad "1" smd roundrect (at -0.95 0) (size 1 1.45) (layers "F.Cu" "F.Mask" "F.Paste") (roundrect_rratio 0.25) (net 2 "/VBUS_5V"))
  (pad "2" smd roundrect (at 0.95 0) (size 1 1.45) (layers "F.Cu" "F.Mask" "F.Paste") (roundrect_rratio 0.25) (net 1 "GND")))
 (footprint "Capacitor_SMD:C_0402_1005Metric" (layer "F.Cu") (at 152.88 88.6)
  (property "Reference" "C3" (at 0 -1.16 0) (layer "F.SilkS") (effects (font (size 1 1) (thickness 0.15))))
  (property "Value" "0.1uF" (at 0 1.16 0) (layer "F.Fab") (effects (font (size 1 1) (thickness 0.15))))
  (fp_line (start -0.107836 -0.36) (end 0.107836 -0.36) (stroke (width 0.12) (type solid)) (layer "F.SilkS"))
  (fp_line (start -0.107836 0.36) (end 0.107836 0.36) (stroke (width 0.12) (type solid)) (layer "F.SilkS"))
  (pad "1" smd roundrect (at -0.48 0) (size 0.56 0.62) (layers "F.Cu" "F.Mask" "F.Paste") (roundrect_rratio 0.25) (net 9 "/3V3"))
  (pad "2" smd roundrect (at 0.48 0) (size 0.56 0.62) (layers "F.Cu" "F.Mask" "F.Paste") (roundrect_rratio 0.25) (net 1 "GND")))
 (gr_rect (start 137.275 86.475) (end 173.275 132.475) (stroke (width 0.05) (type solid)) (fill no) (layer "Edge.Cuts"))
 (segment (start 171.55 87.625) (end 169.89 87.625) (width 0.2) (layer "F.Cu") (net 1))
 (segment (start 167.19 88.975) (end 168.54 88.975) (width 0.2) (layer "F.Cu") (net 1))
 (segment (start 169.89 87.625) (end 168.54 88.975) (width 0.2) (layer "F.Cu") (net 1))
 (segment (start 171.55 96.275) (end 169.89 96.275) (width 0.2) (layer "F.Cu") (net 1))
 (segment (start 168.17 88.605) (end 168.54 88.975) (width 0.2) (layer "F.Cu") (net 1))
 (segment (start 169.89 96.275) (end 168.54 94.925) (width 0.2) (layer "F.Cu") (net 1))
 (segment (start 168.17 95.295) (end 168.54 94.925) (width 0.2) (layer "F.Cu") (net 1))
 (segment (start 168.17 87.625) (end 168.17 88.605) (width 0.2) (layer "F.Cu") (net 1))
 (segment (start 167.19 88.975) (end 162.71 88.975) (width 0.2) (layer "F.Cu") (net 1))
 (segment (start 168.17 96.275) (end 168.17 95.295) (width 0.2) (layer "F.Cu") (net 1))
 (segment (start 162.71 88.975) (end 161.81 89.875) (width 0.2) (layer "F.Cu") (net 1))
 (segment (start 167.19 94.925) (end 168.54 94.925) (width 0.2) (layer "F.Cu") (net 1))
 (segment (start 167.19 89.825) (end 168.54 89.825) (width 0.2) (layer "F.Cu") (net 2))
 (segment (start 168.54 94.075) (end 169.091 93.524) (width 0.2) (layer "F.Cu") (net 2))
 (segment (start 169.091 93.524) (end 169.091 90.376) (width 0.2) (layer "F.Cu") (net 2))
 (segment (start 169.091 90.376) (end 168.54 89.825) (width 0.2) (layer "F.Cu") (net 2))
 (segment (start 167.19 94.075) (end 168.54 94.075) (width 0.2) (layer "F.Cu") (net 2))
 (segment (start 151.326 98.061502) (end 150.939498 97.675) (width 0.2) (layer "F.Cu") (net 11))
 (segment (start 150.939498 97.675) (end 150.2375 97.675) (width 0.2) (layer "F.Cu") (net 11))
 (segment (start 151.326 105.651) (end 151.326 98.061502) (width 0.2) (layer "F.Cu") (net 11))
 (segment (start 168.15 122.475) (end 151.326 105.651) (width 0.2) (layer "F.Cu") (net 11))
 (segment (start 167.19 91.525) (end 164.29 94.425) (width 0.2) (layer "F.Cu") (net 5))
 (segment (start 168.04 92.375) (end 167.19 91.525) (width 0.2) (layer "F.Cu") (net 5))
 (segment (start 168.54 92.375) (end 168.04 92.375) (width 0.2) (layer "F.Cu") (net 5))
 (segment (start 164.29 94.425) (end 157.0625 94.425) (width 0.2) (layer "F.Cu") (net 5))
 (segment (start 168.54 91.525) (end 168.095585 91.525) (width 0.2) (layer "F.Cu") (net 4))
 (segment (start 168.095585 91.525) (end 167.918889 91.348304) (width 0.2) (layer "F.Cu") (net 4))
 (via (at 167.918889 91.348304) (size 0.6) (drill 0.3) (layers "F.Cu" "B.Cu") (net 4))
 (segment (start 167.918889 91.348304) (end 167.918889 91.646111) (width 0.2) (layer "B.Cu") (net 4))
 (segment (start 167.918889 91.646111) (end 167.19 92.375) (width 0.2) (layer "B.Cu") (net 4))
 (segment (start 168.15 119.975) (end 151.627 103.452) (width 0.2) (layer "F.Cu") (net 12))
 (segment (start 151.627 103.452) (end 151.627 97.712502) (width 0.2) (layer "F.Cu") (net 12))
 (segment (start 150.939498 97.025) (end 150.2375 97.025) (width 0.2) (layer "F.Cu") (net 12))
 (segment (start 151.627 97.712502) (end 150.939498 97.025) (width 0.2) (layer "F.Cu") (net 12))
 (segment (start 149.149 105.974) (end 149.149 98.711502) (width 0.2) (layer "F.Cu") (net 16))
 (segment (start 149.149 98.711502) (end 149.535502 98.325) (width 0.2) (layer "F.Cu") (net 16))
 (segment (start 149.535502 98.325) (end 150.2375 98.325) (width 0.2) (layer "F.Cu") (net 16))
 (segment (start 168.15 124.975) (end 149.149 105.974) (width 0.2) (layer "F.Cu") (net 16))
 (segment (start 161.5 91.8) (end 160.5 91.8) (width 0.2) (layer "F.Cu") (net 7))
 (segment (start 167.965928 90.675) (end 167.939536 90.648608) (width 0.2) (layer "F.Cu") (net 7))
 (segment (start 160.5 91.8) (end 159.2 93.1) (width 0.2) (layer "F.Cu") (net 7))
 (segment (start 168.54 90.675) (end 167.965928 90.675) (width 0.2) (layer "F.Cu") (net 7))
 (via (at 167.939536 90.648608) (size 0.6) (drill 0.3) (layers "F.Cu" "B.Cu") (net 7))
 (via (at 161.5 91.8) (size 0.6) (drill 0.3) (layers "F.Cu" "B.Cu") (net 7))
 (segment (start 167.939536 90.648608) (end 167.939536 88.945304) (width 0.2) (layer "B.Cu") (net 7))
 (segment (start 167.418232 88.424) (end 164.876 88.424) (width 0.2) (layer "B.Cu") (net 7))
 (segment (start 164.876 88.424) (end 161.5 91.8) (width 0.2) (layer "B.Cu") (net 7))
 (segment (start 167.939536 88.945304) (end 167.418232 88.424) (width 0.2) (layer "B.Cu") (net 7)))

